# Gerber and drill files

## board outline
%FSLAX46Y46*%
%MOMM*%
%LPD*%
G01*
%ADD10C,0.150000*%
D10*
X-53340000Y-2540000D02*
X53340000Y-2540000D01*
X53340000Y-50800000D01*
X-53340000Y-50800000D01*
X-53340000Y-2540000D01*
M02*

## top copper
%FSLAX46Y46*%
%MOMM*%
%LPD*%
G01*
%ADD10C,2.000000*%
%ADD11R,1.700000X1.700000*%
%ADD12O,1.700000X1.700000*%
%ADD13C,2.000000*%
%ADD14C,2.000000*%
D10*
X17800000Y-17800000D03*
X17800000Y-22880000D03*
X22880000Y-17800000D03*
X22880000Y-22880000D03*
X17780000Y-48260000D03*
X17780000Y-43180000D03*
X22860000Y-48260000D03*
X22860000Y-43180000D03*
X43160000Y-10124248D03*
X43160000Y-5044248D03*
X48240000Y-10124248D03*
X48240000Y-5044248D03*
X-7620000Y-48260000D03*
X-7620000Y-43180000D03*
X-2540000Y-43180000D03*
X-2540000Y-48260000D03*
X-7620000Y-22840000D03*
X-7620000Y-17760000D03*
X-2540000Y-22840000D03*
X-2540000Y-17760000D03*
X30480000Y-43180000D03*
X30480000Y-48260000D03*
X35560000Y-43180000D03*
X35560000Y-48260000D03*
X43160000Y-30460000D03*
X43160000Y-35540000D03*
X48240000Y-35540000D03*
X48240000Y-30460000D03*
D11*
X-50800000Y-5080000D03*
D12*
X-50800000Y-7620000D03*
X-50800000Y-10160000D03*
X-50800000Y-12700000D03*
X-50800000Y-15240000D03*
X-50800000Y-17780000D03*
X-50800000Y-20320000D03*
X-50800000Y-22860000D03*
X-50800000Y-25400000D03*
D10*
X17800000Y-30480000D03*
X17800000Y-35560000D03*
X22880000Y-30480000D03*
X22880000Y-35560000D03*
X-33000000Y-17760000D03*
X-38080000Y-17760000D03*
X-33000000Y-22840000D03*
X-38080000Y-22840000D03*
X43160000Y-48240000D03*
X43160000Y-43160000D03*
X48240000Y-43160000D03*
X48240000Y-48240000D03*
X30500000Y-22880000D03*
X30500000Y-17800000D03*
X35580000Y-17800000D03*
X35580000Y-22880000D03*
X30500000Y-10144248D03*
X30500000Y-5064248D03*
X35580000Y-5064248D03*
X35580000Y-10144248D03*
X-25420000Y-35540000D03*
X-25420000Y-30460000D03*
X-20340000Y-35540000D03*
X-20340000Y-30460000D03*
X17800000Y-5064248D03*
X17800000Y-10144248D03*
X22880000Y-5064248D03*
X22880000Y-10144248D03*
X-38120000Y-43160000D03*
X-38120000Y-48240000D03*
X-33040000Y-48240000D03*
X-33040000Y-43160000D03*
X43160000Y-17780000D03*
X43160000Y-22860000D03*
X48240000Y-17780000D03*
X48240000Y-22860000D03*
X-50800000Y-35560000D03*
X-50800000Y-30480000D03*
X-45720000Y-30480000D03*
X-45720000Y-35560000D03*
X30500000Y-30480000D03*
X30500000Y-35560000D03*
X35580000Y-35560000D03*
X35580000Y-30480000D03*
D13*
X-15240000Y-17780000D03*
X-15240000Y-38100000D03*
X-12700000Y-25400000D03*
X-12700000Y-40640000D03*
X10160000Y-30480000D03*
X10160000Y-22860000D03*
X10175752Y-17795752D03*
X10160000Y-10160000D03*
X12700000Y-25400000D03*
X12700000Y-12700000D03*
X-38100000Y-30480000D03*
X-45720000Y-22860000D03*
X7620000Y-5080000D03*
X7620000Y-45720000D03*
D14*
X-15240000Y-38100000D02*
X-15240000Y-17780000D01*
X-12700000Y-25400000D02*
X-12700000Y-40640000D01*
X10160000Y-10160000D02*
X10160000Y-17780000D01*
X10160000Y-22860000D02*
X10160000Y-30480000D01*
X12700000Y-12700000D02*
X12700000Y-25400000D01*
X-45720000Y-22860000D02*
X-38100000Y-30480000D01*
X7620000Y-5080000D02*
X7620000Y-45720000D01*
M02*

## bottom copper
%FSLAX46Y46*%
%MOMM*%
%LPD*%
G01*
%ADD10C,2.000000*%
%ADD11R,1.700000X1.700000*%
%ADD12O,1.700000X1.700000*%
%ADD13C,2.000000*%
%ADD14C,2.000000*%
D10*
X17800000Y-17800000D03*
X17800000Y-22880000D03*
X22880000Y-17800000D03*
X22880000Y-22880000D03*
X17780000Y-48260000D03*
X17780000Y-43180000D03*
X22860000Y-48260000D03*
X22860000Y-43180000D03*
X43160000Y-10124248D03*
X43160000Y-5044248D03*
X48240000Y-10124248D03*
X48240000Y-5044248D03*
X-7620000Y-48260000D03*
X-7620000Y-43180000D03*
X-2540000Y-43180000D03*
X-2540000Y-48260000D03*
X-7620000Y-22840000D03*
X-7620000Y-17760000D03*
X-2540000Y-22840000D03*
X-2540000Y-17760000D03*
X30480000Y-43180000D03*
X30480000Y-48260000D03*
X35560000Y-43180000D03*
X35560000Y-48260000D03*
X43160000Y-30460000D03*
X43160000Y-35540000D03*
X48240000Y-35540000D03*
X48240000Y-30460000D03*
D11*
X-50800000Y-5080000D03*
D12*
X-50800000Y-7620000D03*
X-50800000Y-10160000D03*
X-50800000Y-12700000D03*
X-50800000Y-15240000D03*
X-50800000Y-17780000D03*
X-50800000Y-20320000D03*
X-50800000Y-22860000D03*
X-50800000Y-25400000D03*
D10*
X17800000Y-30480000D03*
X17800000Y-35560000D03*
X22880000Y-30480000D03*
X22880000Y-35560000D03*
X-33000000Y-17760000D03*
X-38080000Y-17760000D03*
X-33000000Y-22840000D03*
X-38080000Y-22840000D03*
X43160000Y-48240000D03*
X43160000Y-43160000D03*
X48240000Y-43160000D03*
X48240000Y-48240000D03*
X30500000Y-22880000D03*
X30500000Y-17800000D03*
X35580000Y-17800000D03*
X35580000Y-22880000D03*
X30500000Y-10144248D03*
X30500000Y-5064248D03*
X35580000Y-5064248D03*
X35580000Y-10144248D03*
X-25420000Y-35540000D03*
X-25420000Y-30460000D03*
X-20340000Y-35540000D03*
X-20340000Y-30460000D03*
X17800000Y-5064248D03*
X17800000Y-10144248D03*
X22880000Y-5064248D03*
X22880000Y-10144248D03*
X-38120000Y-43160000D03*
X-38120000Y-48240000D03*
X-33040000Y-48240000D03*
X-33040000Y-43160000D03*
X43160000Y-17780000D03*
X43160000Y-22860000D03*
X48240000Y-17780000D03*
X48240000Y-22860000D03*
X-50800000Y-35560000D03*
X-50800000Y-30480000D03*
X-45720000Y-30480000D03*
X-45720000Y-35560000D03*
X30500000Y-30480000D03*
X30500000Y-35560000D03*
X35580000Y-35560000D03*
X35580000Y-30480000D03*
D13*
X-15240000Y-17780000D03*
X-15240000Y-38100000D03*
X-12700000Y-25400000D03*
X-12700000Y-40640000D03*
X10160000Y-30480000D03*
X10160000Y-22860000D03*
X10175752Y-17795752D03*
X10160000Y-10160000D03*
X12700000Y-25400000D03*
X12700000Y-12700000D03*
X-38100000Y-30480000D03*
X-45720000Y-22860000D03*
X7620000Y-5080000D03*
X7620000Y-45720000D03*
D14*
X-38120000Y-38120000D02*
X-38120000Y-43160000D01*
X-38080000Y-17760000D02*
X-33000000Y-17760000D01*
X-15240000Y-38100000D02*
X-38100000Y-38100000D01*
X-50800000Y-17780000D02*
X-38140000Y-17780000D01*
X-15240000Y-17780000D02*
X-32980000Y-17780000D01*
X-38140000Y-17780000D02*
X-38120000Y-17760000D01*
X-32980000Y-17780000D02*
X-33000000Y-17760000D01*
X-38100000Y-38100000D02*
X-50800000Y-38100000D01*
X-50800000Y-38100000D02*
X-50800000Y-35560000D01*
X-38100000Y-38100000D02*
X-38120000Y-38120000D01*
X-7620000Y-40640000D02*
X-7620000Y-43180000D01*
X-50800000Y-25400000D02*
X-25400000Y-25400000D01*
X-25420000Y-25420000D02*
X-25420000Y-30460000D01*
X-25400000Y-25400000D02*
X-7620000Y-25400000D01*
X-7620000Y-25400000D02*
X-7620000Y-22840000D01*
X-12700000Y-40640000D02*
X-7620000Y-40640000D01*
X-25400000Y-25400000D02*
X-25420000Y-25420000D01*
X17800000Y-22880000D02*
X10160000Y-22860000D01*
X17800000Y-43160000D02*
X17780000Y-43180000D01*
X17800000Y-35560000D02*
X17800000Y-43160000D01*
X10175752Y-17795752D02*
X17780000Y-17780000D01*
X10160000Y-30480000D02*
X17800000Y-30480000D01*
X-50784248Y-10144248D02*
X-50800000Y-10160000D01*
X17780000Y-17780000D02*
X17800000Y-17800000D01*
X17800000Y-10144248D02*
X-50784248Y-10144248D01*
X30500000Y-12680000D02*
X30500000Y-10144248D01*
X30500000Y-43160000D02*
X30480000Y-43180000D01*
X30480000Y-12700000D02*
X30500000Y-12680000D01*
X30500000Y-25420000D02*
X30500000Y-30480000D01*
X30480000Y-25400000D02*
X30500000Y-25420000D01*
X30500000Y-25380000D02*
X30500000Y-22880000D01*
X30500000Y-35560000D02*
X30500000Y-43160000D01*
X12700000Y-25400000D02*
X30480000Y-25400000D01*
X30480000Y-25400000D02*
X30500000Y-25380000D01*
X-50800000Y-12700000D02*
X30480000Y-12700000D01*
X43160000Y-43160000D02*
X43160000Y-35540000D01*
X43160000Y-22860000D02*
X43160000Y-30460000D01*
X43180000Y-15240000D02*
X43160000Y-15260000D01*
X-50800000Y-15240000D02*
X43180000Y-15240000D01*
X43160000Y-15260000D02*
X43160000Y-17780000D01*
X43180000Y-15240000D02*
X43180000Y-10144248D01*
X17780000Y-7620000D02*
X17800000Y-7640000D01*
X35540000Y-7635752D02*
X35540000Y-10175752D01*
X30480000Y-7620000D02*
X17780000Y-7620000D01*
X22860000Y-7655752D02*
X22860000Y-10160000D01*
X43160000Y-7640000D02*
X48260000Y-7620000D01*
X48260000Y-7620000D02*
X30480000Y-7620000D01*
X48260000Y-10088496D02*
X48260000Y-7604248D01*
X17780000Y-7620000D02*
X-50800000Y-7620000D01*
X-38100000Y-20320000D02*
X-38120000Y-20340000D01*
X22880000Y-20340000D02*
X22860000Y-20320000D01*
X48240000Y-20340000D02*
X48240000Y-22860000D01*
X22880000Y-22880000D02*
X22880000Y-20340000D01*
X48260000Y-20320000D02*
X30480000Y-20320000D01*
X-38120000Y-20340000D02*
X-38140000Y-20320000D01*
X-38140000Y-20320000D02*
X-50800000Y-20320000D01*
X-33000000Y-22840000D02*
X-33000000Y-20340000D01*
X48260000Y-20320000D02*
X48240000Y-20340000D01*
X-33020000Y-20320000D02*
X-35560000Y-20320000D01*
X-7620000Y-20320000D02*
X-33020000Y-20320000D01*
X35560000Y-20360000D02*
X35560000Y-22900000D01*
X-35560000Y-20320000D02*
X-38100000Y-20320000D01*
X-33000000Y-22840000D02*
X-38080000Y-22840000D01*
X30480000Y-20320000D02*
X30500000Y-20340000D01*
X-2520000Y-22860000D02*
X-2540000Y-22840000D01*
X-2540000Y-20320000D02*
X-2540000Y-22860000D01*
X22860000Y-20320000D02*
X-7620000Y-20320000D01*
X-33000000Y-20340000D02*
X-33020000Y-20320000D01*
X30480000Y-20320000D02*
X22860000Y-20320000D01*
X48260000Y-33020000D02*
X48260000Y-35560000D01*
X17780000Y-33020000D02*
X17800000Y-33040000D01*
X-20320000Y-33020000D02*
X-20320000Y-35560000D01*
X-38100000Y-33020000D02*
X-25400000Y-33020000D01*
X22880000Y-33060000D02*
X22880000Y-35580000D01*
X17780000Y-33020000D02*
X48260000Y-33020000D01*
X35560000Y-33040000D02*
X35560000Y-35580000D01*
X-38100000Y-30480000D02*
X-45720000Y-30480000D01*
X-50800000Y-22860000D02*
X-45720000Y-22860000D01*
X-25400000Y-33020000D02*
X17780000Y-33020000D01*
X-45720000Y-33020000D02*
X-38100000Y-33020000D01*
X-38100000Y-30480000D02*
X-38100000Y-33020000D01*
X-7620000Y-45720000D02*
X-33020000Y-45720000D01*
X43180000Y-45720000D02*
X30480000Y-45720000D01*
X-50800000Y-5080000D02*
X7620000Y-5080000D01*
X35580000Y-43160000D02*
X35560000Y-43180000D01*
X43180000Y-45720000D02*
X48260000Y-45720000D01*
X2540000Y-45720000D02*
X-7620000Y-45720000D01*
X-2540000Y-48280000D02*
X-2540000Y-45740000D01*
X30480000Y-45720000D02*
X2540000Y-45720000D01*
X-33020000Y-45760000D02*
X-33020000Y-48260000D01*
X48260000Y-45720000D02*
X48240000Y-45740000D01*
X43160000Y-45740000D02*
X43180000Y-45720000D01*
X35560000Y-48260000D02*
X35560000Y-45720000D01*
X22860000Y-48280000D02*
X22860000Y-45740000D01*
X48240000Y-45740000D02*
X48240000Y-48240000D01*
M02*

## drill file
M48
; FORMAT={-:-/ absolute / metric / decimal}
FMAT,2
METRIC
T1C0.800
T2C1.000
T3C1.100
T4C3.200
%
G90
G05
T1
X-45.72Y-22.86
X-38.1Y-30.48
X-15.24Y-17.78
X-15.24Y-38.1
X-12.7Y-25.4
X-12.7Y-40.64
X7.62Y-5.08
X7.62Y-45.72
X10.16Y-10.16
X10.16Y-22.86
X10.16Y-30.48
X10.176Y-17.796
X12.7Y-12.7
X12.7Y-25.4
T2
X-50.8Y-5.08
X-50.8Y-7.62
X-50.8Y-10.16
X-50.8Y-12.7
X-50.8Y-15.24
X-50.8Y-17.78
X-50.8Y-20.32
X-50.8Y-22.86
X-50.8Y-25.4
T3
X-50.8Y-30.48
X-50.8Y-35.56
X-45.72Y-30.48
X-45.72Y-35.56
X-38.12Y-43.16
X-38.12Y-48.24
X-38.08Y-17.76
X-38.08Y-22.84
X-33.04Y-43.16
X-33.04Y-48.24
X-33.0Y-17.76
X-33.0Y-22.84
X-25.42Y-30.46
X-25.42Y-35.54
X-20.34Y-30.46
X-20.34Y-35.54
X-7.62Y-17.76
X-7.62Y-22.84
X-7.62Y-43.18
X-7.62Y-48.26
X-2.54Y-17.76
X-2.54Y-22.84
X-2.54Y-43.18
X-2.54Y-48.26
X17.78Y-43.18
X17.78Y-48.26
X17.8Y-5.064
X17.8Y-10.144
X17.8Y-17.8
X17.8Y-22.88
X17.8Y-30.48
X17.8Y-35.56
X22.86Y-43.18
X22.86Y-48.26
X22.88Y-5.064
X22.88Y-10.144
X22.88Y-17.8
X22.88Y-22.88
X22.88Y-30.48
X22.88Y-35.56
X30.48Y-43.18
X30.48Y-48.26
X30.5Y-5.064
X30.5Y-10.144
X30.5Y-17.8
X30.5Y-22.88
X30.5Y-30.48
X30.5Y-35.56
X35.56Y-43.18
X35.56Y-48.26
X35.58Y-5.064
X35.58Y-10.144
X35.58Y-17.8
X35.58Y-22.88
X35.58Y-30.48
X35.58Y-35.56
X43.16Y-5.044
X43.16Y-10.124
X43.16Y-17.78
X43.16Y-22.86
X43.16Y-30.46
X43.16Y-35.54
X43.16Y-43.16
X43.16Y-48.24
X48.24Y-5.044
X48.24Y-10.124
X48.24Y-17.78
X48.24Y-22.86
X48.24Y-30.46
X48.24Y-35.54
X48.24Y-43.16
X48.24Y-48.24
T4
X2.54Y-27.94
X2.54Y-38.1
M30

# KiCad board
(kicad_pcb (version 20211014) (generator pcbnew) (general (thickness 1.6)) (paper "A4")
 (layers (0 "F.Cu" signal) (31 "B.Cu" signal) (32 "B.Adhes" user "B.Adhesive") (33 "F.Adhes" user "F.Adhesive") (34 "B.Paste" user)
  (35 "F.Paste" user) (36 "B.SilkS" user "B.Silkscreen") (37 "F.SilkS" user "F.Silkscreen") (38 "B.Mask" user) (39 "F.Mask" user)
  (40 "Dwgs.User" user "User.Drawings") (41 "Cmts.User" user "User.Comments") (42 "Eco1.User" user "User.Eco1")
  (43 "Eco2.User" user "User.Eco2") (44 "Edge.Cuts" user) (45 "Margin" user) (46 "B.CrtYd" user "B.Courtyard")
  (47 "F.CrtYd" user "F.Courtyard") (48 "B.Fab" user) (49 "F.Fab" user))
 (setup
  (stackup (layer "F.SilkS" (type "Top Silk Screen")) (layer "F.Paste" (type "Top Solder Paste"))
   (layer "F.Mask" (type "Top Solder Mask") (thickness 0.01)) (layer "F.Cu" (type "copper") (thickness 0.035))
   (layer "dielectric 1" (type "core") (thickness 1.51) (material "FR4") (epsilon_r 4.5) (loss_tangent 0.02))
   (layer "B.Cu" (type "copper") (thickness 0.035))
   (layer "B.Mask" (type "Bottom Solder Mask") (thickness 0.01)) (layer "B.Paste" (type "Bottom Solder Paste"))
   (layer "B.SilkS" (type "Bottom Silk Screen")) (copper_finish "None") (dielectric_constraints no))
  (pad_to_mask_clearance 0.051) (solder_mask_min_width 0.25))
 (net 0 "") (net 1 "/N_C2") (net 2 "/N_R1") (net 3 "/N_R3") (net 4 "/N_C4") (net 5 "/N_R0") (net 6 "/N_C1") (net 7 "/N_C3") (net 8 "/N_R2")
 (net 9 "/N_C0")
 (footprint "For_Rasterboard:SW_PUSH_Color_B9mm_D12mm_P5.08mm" (layer "F.Cu") (at 17.8 17.8)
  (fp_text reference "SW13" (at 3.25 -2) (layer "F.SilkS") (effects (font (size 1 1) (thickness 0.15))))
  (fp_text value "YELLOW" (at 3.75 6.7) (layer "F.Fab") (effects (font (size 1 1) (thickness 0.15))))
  (pad "1" thru_hole circle (at 0 0 90) (size 2 2) (drill 1.1) (layers *.Cu *.Mask) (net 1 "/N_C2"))
  (pad "1" thru_hole circle (at 0 5.08 90) (size 2 2) (drill 1.1) (layers *.Cu *.Mask) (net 1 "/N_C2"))
  (pad "2" thru_hole circle (at 5.08 0 90) (size 2 2) (drill 1.1) (layers *.Cu *.Mask) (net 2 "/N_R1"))
  (pad "2" thru_hole circle (at 5.08 5.08 180) (size 2 2) (drill 1.1) (layers *.Cu *.Mask) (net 2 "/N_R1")))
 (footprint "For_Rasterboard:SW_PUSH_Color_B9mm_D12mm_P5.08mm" (layer "F.Cu") (at 17.78 43.18)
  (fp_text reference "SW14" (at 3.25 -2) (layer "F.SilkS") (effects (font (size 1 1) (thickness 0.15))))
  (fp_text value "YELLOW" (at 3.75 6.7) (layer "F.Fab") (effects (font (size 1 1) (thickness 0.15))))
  (pad "1" thru_hole circle (at 0 5.08 90) (size 2 2) (drill 1.1) (layers *.Cu *.Mask) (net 1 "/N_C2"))
  (pad "1" thru_hole circle (at 0 0 90) (size 2 2) (drill 1.1) (layers *.Cu *.Mask) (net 1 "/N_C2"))
  (pad "2" thru_hole circle (at 5.08 5.08 180) (size 2 2) (drill 1.1) (layers *.Cu *.Mask) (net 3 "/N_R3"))
  (pad "2" thru_hole circle (at 5.08 0 90) (size 2 2) (drill 1.1) (layers *.Cu *.Mask) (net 3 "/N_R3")))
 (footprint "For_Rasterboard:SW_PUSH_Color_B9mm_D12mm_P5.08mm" (layer "F.Cu") (at 43.16 5.044248)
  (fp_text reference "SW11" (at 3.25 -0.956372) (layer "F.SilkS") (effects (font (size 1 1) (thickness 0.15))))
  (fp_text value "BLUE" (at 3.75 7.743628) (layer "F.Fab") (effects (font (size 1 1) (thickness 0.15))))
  (pad "1" thru_hole circle (at 0 5.08 90) (size 2 2) (drill 1.1) (layers *.Cu *.Mask) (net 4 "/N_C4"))
  (pad "1" thru_hole circle (at 0 0 90) (size 2 2) (drill 1.1) (layers *.Cu *.Mask) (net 4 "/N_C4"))
  (pad "2" thru_hole circle (at 5.08 5.08 180) (size 2 2) (drill 1.1) (layers *.Cu *.Mask) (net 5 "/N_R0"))
  (pad "2" thru_hole circle (at 5.08 0 90) (size 2 2) (drill 1.1) (layers *.Cu *.Mask) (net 5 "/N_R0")))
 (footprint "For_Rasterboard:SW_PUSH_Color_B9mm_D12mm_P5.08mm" (layer "F.Cu") (at -7.62 43.18)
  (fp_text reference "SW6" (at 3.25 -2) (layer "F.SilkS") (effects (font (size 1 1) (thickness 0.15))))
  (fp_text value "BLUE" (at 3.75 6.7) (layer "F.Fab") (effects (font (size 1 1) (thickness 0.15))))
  (pad "1" thru_hole circle (at 0 5.08 90) (size 2 2) (drill 1.1) (layers *.Cu *.Mask) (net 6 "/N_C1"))
  (pad "1" thru_hole circle (at 0 0 90) (size 2 2) (drill 1.1) (layers *.Cu *.Mask) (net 6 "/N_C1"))
  (pad "2" thru_hole circle (at 5.08 0 90) (size 2 2) (drill 1.1) (layers *.Cu *.Mask) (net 3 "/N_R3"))
  (pad "2" thru_hole circle (at 5.08 5.08 180) (size 2 2) (drill 1.1) (layers *.Cu *.Mask) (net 3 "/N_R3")))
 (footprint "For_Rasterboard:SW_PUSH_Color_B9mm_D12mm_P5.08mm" (layer "F.Cu") (at -7.62 17.76)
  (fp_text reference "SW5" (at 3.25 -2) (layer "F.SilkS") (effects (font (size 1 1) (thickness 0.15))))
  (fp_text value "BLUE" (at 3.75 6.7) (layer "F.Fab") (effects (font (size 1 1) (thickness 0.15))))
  (pad "1" thru_hole circle (at 0 5.08 90) (size 2 2) (drill 1.1) (layers *.Cu *.Mask) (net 6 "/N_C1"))
  (pad "1" thru_hole circle (at 0 0 90) (size 2 2) (drill 1.1) (layers *.Cu *.Mask) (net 6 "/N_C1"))
  (pad "2" thru_hole circle (at 5.08 5.08 180) (size 2 2) (drill 1.1) (layers *.Cu *.Mask) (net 2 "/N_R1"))
  (pad "2" thru_hole circle (at 5.08 0 90) (size 2 2) (drill 1.1) (layers *.Cu *.Mask) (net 2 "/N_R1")))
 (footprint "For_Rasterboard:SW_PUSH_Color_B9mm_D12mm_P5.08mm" (layer "F.Cu") (at 30.48 43.18)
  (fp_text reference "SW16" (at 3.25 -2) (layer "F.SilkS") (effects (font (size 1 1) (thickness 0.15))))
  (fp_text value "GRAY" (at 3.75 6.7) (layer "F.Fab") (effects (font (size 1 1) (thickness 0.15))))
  (pad "1" thru_hole circle (at 0 0 90) (size 2 2) (drill 1.1) (layers *.Cu *.Mask) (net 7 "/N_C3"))
  (pad "1" thru_hole circle (at 0 5.08 90) (size 2 2) (drill 1.1) (layers *.Cu *.Mask) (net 7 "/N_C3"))
  (pad "2" thru_hole circle (at 5.08 0 90) (size 2 2) (drill 1.1) (layers *.Cu *.Mask) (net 3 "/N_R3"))
  (pad "2" thru_hole circle (at 5.08 5.08 180) (size 2 2) (drill 1.1) (layers *.Cu *.Mask) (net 3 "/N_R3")))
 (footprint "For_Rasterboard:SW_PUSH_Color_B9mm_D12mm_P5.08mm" (layer "F.Cu") (at 43.16 30.46)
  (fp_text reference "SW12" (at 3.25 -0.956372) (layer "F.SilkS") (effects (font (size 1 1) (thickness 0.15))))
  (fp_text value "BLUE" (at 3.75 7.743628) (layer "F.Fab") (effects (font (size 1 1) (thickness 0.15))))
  (pad "1" thru_hole circle (at 0 0 90) (size 2 2) (drill 1.1) (layers *.Cu *.Mask) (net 4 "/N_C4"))
  (pad "1" thru_hole circle (at 0 5.08 90) (size 2 2) (drill 1.1) (layers *.Cu *.Mask) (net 4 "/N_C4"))
  (pad "2" thru_hole circle (at 5.08 5.08 180) (size 2 2) (drill 1.1) (layers *.Cu *.Mask) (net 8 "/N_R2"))
  (pad "2" thru_hole circle (at 5.08 0 90) (size 2 2) (drill 1.1) (layers *.Cu *.Mask) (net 8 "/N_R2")))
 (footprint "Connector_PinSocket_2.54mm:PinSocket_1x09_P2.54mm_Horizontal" (layer "F.Cu") (at -50.8 5.08)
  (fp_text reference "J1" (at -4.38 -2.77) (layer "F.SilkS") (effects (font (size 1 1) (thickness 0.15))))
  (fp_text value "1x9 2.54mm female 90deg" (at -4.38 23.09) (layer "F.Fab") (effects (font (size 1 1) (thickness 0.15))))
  (pad "1" thru_hole rect (at 0 0) (size 1.7 1.7) (drill 1) (layers *.Cu *.Mask) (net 3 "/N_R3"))
  (pad "2" thru_hole oval (at 0 2.54) (size 1.7 1.7) (drill 1) (layers *.Cu *.Mask) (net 5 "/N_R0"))
  (pad "3" thru_hole oval (at 0 5.08) (size 1.7 1.7) (drill 1) (layers *.Cu *.Mask) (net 1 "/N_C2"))
  (pad "4" thru_hole oval (at 0 7.62) (size 1.7 1.7) (drill 1) (layers *.Cu *.Mask) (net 7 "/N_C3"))
  (pad "5" thru_hole oval (at 0 10.16) (size 1.7 1.7) (drill 1) (layers *.Cu *.Mask) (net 4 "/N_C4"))
  (pad "6" thru_hole oval (at 0 12.7) (size 1.7 1.7) (drill 1) (layers *.Cu *.Mask) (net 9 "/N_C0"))
  (pad "7" thru_hole oval (at 0 15.24) (size 1.7 1.7) (drill 1) (layers *.Cu *.Mask) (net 2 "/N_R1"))
  (pad "8" thru_hole oval (at 0 17.78) (size 1.7 1.7) (drill 1) (layers *.Cu *.Mask) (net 8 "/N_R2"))
  (pad "9" thru_hole oval (at 0 20.32) (size 1.7 1.7) (drill 1) (layers *.Cu *.Mask) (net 6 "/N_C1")))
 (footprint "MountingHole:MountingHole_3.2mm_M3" (layer "F.Cu") (at 2.54 27.94)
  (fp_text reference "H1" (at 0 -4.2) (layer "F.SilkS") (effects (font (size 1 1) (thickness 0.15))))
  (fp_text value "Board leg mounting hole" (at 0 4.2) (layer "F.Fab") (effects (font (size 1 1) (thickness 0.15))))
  (pad "" np_thru_hole circle (at 0 0) (size 3.2 3.2) (drill 3.2) (layers *.Cu *.Mask)))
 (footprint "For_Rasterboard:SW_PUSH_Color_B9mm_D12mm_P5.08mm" (layer "F.Cu") (at 17.8 30.48)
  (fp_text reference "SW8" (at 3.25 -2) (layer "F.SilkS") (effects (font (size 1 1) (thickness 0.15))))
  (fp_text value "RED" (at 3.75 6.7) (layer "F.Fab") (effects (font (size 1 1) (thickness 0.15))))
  (pad "1" thru_hole circle (at 0 0 90) (size 2 2) (drill 1.1) (layers *.Cu *.Mask) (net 1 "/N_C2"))
  (pad "1" thru_hole circle (at 0 5.08 90) (size 2 2) (drill 1.1) (layers *.Cu *.Mask) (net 1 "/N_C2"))
  (pad "2" thru_hole circle (at 5.08 0 90) (size 2 2) (drill 1.1) (layers *.Cu *.Mask) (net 8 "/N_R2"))
  (pad "2" thru_hole circle (at 5.08 5.08 180) (size 2 2) (drill 1.1) (layers *.Cu *.Mask) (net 8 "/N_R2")))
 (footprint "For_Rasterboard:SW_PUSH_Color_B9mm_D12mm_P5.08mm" (layer "F.Cu") (at -33 17.76 -90)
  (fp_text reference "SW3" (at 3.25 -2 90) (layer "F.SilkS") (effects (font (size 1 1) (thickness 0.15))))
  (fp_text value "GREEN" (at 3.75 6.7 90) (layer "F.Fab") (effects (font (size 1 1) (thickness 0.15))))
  (pad "1" thru_hole circle (at 0 0) (size 2 2) (drill 1.1) (layers *.Cu *.Mask) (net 9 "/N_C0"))
  (pad "1" thru_hole circle (at 0 5.08) (size 2 2) (drill 1.1) (layers *.Cu *.Mask) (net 9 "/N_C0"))
  (pad "2" thru_hole circle (at 5.08 0) (size 2 2) (drill 1.1) (layers *.Cu *.Mask) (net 2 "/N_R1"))
  (pad "2" thru_hole circle (at 5.08 5.08 90) (size 2 2) (drill 1.1) (layers *.Cu *.Mask) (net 2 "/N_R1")))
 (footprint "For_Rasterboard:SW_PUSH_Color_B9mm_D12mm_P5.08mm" (layer "F.Cu") (at 43.16 43.16)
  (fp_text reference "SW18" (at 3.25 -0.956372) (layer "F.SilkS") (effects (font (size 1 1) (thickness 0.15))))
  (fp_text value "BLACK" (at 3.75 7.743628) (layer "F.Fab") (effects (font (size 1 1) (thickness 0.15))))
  (pad "1" thru_hole circle (at 0 5.08 90) (size 2 2) (drill 1.1) (layers *.Cu *.Mask) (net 4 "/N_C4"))
  (pad "1" thru_hole circle (at 0 0 90) (size 2 2) (drill 1.1) (layers *.Cu *.Mask) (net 4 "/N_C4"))
  (pad "2" thru_hole circle (at 5.08 0 90) (size 2 2) (drill 1.1) (layers *.Cu *.Mask) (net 3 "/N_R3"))
  (pad "2" thru_hole circle (at 5.08 5.08 180) (size 2 2) (drill 1.1) (layers *.Cu *.Mask) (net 3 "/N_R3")))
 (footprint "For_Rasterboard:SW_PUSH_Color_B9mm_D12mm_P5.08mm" (layer "F.Cu") (at 30.5 17.8)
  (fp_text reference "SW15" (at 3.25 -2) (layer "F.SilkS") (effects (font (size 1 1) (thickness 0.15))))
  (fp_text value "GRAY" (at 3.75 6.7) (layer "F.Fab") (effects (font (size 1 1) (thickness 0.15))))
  (pad "1" thru_hole circle (at 0 5.08 90) (size 2 2) (drill 1.1) (layers *.Cu *.Mask) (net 7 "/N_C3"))
  (pad "1" thru_hole circle (at 0 0 90) (size 2 2) (drill 1.1) (layers *.Cu *.Mask) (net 7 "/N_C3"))
  (pad "2" thru_hole circle (at 5.08 0 90) (size 2 2) (drill 1.1) (layers *.Cu *.Mask) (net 2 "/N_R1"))
  (pad "2" thru_hole circle (at 5.08 5.08 180) (size 2 2) (drill 1.1) (layers *.Cu *.Mask) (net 2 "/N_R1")))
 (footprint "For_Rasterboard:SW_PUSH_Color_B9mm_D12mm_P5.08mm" (layer "F.Cu") (at 30.5 5.064248)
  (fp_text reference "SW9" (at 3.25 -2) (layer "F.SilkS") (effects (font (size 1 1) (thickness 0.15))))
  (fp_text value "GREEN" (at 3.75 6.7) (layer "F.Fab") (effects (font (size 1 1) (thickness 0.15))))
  (pad "1" thru_hole circle (at 0 5.08 90) (size 2 2) (drill 1.1) (layers *.Cu *.Mask) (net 7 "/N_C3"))
  (pad "1" thru_hole circle (at 0 0 90) (size 2 2) (drill 1.1) (layers *.Cu *.Mask) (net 7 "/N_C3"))
  (pad "2" thru_hole circle (at 5.08 0 90) (size 2 2) (drill 1.1) (layers *.Cu *.Mask) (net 5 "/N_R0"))
  (pad "2" thru_hole circle (at 5.08 5.08 180) (size 2 2) (drill 1.1) (layers *.Cu *.Mask) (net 5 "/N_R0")))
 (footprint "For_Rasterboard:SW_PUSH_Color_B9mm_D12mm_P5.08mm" (layer "F.Cu") (at -25.42 30.46)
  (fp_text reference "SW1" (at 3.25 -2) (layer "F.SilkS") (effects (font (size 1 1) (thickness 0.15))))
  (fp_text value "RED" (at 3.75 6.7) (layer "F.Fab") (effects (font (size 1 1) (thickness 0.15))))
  (pad "1" thru_hole circle (at 0 5.08 90) (size 2 2) (drill 1.1) (layers *.Cu *.Mask) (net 6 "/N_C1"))
  (pad "1" thru_hole circle (at 0 0 90) (size 2 2) (drill 1.1) (layers *.Cu *.Mask) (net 6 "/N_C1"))
  (pad "2" thru_hole circle (at 5.08 5.08 180) (size 2 2) (drill 1.1) (layers *.Cu *.Mask) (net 8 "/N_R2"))
  (pad "2" thru_hole circle (at 5.08 0 90) (size 2 2) (drill 1.1) (layers *.Cu *.Mask) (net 8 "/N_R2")))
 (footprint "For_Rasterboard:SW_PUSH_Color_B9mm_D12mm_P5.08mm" (layer "F.Cu") (at 17.8 5.064248)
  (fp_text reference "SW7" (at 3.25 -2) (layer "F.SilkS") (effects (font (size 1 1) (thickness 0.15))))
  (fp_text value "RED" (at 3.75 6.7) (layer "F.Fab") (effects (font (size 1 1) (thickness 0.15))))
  (pad "1" thru_hole circle (at 0 0 90) (size 2 2) (drill 1.1) (layers *.Cu *.Mask) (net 1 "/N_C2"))
  (pad "1" thru_hole circle (at 0 5.08 90) (size 2 2) (drill 1.1) (layers *.Cu *.Mask) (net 1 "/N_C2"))
  (pad "2" thru_hole circle (at 5.08 0 90) (size 2 2) (drill 1.1) (layers *.Cu *.Mask) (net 5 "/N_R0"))
  (pad "2" thru_hole circle (at 5.08 5.08 180) (size 2 2) (drill 1.1) (layers *.Cu *.Mask) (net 5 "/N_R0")))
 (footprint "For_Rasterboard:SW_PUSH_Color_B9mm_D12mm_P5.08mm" (layer "F.Cu") (at -38.12 43.16)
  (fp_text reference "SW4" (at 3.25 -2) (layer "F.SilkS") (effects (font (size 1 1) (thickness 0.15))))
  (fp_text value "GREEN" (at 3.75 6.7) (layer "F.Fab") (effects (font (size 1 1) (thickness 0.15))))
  (pad "1" thru_hole circle (at 0 0 90) (size 2 2) (drill 1.1) (layers *.Cu *.Mask) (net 9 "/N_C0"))
  (pad "1" thru_hole circle (at 0 5.08 90) (size 2 2) (drill 1.1) (layers *.Cu *.Mask) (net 9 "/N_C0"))
  (pad "2" thru_hole circle (at 5.08 5.08 180) (size 2 2) (drill 1.1) (layers *.Cu *.Mask) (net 3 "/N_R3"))
  (pad "2" thru_hole circle (at 5.08 0 90) (size 2 2) (drill 1.1) (layers *.Cu *.Mask) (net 3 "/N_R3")))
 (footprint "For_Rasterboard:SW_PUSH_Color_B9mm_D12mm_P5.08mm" (layer "F.Cu") (at 43.16 17.78)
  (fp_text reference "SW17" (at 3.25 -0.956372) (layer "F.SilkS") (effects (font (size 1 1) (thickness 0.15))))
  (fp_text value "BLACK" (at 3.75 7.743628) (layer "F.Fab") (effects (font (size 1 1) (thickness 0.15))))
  (pad "1" thru_hole circle (at 0 0 90) (size 2 2) (drill 1.1) (layers *.Cu *.Mask) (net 4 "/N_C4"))
  (pad "1" thru_hole circle (at 0 5.08 90) (size 2 2) (drill 1.1) (layers *.Cu *.Mask) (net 4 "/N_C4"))
  (pad "2" thru_hole circle (at 5.08 0 90) (size 2 2) (drill 1.1) (layers *.Cu *.Mask) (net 2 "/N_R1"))
  (pad "2" thru_hole circle (at 5.08 5.08 180) (size 2 2) (drill 1.1) (layers *.Cu *.Mask) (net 2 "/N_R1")))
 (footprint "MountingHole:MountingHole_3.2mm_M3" (layer "F.Cu") (at 2.54 38.1)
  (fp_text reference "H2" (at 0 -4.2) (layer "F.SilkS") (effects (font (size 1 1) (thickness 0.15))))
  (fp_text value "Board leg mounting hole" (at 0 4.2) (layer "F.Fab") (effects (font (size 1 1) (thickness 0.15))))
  (pad "" np_thru_hole circle (at 0 0) (size 3.2 3.2) (drill 3.2) (layers *.Cu *.Mask)))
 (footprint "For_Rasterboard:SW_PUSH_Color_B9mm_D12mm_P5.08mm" (layer "F.Cu") (at -50.8 30.48)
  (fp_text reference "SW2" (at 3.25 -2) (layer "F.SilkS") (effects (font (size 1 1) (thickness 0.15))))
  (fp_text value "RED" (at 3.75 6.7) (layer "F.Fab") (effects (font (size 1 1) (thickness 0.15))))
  (pad "1" thru_hole circle (at 0 5.08 90) (size 2 2) (drill 1.1) (layers *.Cu *.Mask) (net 9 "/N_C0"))
  (pad "1" thru_hole circle (at 0 0 90) (size 2 2) (drill 1.1) (layers *.Cu *.Mask) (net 9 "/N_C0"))
  (pad "2" thru_hole circle (at 5.08 0 90) (size 2 2) (drill 1.1) (layers *.Cu *.Mask) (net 8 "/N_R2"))
  (pad "2" thru_hole circle (at 5.08 5.08 180) (size 2 2) (drill 1.1) (layers *.Cu *.Mask) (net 8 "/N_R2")))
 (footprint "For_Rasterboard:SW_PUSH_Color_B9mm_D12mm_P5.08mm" (layer "F.Cu") (at 30.5 30.48)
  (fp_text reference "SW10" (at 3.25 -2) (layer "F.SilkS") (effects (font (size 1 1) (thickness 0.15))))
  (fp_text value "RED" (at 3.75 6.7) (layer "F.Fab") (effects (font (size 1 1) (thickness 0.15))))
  (pad "1" thru_hole circle (at 0 0 90) (size 2 2) (drill 1.1) (layers *.Cu *.Mask) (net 7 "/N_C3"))
  (pad "1" thru_hole circle (at 0 5.08 90) (size 2 2) (drill 1.1) (layers *.Cu *.Mask) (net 7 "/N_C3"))
  (pad "2" thru_hole circle (at 5.08 5.08 180) (size 2 2) (drill 1.1) (layers *.Cu *.Mask) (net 8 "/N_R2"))
  (pad "2" thru_hole circle (at 5.08 0 90) (size 2 2) (drill 1.1) (layers *.Cu *.Mask) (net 8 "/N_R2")))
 (gr_rect (start -53.34 2.54) (end 53.34 50.8) (layer "Edge.Cuts") (width 0.15) (fill none))
 (segment (start -15.24 38.1) (end -15.24 17.78) (width 2) (layer "F.Cu") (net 9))
 (via (at -15.24 17.78) (size 2) (drill 0.8) (layers "F.Cu" "B.Cu") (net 9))
 (via (at -15.24 38.1) (size 2) (drill 0.8) (layers "F.Cu" "B.Cu") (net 9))
 (segment (start -38.12 38.12) (end -38.12 43.16) (width 2) (layer "B.Cu") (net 9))
 (segment (start -38.08 17.76) (end -33 17.76) (width 2) (layer "B.Cu") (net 9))
 (segment (start -15.24 38.1) (end -38.1 38.1) (width 2) (layer "B.Cu") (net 9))
 (segment (start -50.8 17.78) (end -38.14 17.78) (width 2) (layer "B.Cu") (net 9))
 (segment (start -15.24 17.78) (end -32.98 17.78) (width 2) (layer "B.Cu") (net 9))
 (segment (start -38.14 17.78) (end -38.12 17.76) (width 2) (layer "B.Cu") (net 9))
 (segment (start -32.98 17.78) (end -33 17.76) (width 2) (layer "B.Cu") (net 9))
 (segment (start -38.1 38.1) (end -50.8 38.1) (width 2) (layer "B.Cu") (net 9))
 (segment (start -50.8 38.1) (end -50.8 35.56) (width 2) (layer "B.Cu") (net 9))
 (segment (start -38.1 38.1) (end -38.12 38.12) (width 2) (layer "B.Cu") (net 9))
 (segment (start -12.7 25.4) (end -12.7 40.64) (width 2) (layer "F.Cu") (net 6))
 (via (at -12.7 25.4) (size 2) (drill 0.8) (layers "F.Cu" "B.Cu") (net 6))
 (via (at -12.7 40.64) (size 2) (drill 0.8) (layers "F.Cu" "B.Cu") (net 6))
 (segment (start -7.62 40.64) (end -7.62 43.18) (width 2) (layer "B.Cu") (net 6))
 (segment (start -50.8 25.4) (end -25.4 25.4) (width 2) (layer "B.Cu") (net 6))
 (segment (start -25.42 25.42) (end -25.42 30.46) (width 2) (layer "B.Cu") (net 6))
 (segment (start -25.4 25.4) (end -7.62 25.4) (width 2) (layer "B.Cu") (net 6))
 (segment (start -7.62 25.4) (end -7.62 22.84) (width 2) (layer "B.Cu") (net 6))
 (segment (start -12.7 40.64) (end -7.62 40.64) (width 2) (layer "B.Cu") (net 6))
 (segment (start -25.4 25.4) (end -25.42 25.42) (width 2) (layer "B.Cu") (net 6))
 (segment (start 10.16 10.16) (end 10.16 17.78) (width 2) (layer "F.Cu") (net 1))
 (segment (start 10.16 22.86) (end 10.16 30.48) (width 2) (layer "F.Cu") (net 1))
 (via (at 10.16 30.48) (size 2) (drill 0.8) (layers "F.Cu" "B.Cu") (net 1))
 (via (at 10.16 22.86) (size 2) (drill 0.8) (layers "F.Cu" "B.Cu") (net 1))
 (via (at 10.175752 17.795752) (size 2) (drill 0.8) (layers "F.Cu" "B.Cu") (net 1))
 (via (at 10.16 10.16) (size 2) (drill 0.8) (layers "F.Cu" "B.Cu") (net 1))
 (segment (start 17.8 22.88) (end 10.16 22.86) (width 2) (layer "B.Cu") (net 1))
 (segment (start 17.8 43.16) (end 17.78 43.18) (width 2) (layer "B.Cu") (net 1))
 (segment (start 17.8 35.56) (end 17.8 43.16) (width 2) (layer "B.Cu") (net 1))
 (segment (start 10.175752 17.795752) (end 17.78 17.78) (width 2) (layer "B.Cu") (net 1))
 (segment (start 10.16 30.48) (end 17.8 30.48) (width 2) (layer "B.Cu") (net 1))
 (segment (start -50.784248 10.144248) (end -50.8 10.16) (width 2) (layer "B.Cu") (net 1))
 (segment (start 17.78 17.78) (end 17.8 17.8) (width 2) (layer "B.Cu") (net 1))
 (segment (start 17.8 10.144248) (end -50.784248 10.144248) (width 2) (layer "B.Cu") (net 1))
 (segment (start 12.7 12.7) (end 12.7 25.4) (width 2) (layer "F.Cu") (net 7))
 (via (at 12.7 25.4) (size 2) (drill 0.8) (layers "F.Cu" "B.Cu") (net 7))
 (via (at 12.7 12.7) (size 2) (drill 0.8) (layers "F.Cu" "B.Cu") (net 7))
 (segment (start 30.5 12.68) (end 30.5 10.144248) (width 2) (layer "B.Cu") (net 7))
 (segment (start 30.5 43.16) (end 30.48 43.18) (width 2) (layer "B.Cu") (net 7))
 (segment (start 30.48 12.7) (end 30.5 12.68) (width 2) (layer "B.Cu") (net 7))
 (segment (start 30.5 25.42) (end 30.5 30.48) (width 2) (layer "B.Cu") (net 7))
 (segment (start 30.48 25.4) (end 30.5 25.42) (width 2) (layer "B.Cu") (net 7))
 (segment (start 30.5 25.38) (end 30.5 22.88) (width 2) (layer "B.Cu") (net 7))
 (segment (start 30.5 35.56) (end 30.5 43.16) (width 2) (layer "B.Cu") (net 7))
 (segment (start 12.7 25.4) (end 30.48 25.4) (width 2) (layer "B.Cu") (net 7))
 (segment (start 30.48 25.4) (end 30.5 25.38) (width 2) (layer "B.Cu") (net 7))
 (segment (start -50.8 12.7) (end 30.48 12.7) (width 2) (layer "B.Cu") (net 7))
 (segment (start 43.16 43.16) (end 43.16 35.54) (width 2) (layer "B.Cu") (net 4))
 (segment (start 43.16 22.86) (end 43.16 30.46) (width 2) (layer "B.Cu") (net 4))
 (segment (start 43.18 15.24) (end 43.16 15.26) (width 2) (layer "B.Cu") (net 4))
 (segment (start -50.8 15.24) (end 43.18 15.24) (width 2) (layer "B.Cu") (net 4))
 (segment (start 43.16 15.26) (end 43.16 17.78) (width 2) (layer "B.Cu") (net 4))
 (segment (start 43.18 15.24) (end 43.18 10.144248) (width 2) (layer "B.Cu") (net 4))
 (segment (start 17.78 7.62) (end 17.8 7.64) (width 2) (layer "B.Cu") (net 5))
 (segment (start 35.54 7.635752) (end 35.54 10.175752) (width 2) (layer "B.Cu") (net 5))
 (segment (start 30.48 7.62) (end 17.78 7.62) (width 2) (layer "B.Cu") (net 5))
 (segment (start 22.86 7.655752) (end 22.86 10.16) (width 2) (layer "B.Cu") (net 5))
 (segment (start 43.16 7.64) (end 48.26 7.62) (width 2) (layer "B.Cu") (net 5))
 (segment (start 48.26 7.62) (end 30.48 7.62) (width 2) (layer "B.Cu") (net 5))
 (segment (start 48.26 10.088496) (end 48.26 7.604248) (width 2) (layer "B.Cu") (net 5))
 (segment (start 17.78 7.62) (end -50.8 7.62) (width 2) (layer "B.Cu") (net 5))
 (segment (start -38.1 20.32) (end -38.12 20.34) (width 2) (layer "B.Cu") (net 2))
 (segment (start 22.88 20.34) (end 22.86 20.32) (width 2) (layer "B.Cu") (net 2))
 (segment (start 48.24 20.34) (end 48.24 22.86) (width 2) (layer "B.Cu") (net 2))
 (segment (start 22.88 22.88) (end 22.88 20.34) (width 2) (layer "B.Cu") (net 2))
 (segment (start 48.26 20.32) (end 30.48 20.32) (width 2) (layer "B.Cu") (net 2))
 (segment (start -38.12 20.34) (end -38.14 20.32) (width 2) (layer "B.Cu") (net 2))
 (segment (start -38.14 20.32) (end -50.8 20.32) (width 2) (layer "B.Cu") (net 2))
 (segment (start -33 22.84) (end -33 20.34) (width 2) (layer "B.Cu") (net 2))
 (segment (start 48.26 20.32) (end 48.24 20.34) (width 2) (layer "B.Cu") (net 2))
 (segment (start -33.02 20.32) (end -35.56 20.32) (width 2) (layer "B.Cu") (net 2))
 (segment (start -7.62 20.32) (end -33.02 20.32) (width 2) (layer "B.Cu") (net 2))
 (segment (start 35.56 20.36) (end 35.56 22.9) (width 2) (layer "B.Cu") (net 2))
 (segment (start -35.56 20.32) (end -38.1 20.32) (width 2) (layer "B.Cu") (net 2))
 (segment (start -33 22.84) (end -38.08 22.84) (width 2) (layer "B.Cu") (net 2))
 (segment (start 30.48 20.32) (end 30.5 20.34) (width 2) (layer "B.Cu") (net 2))
 (segment (start -2.52 22.86) (end -2.54 22.84) (width 2) (layer "B.Cu") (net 2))
 (segment (start -2.54 20.32) (end -2.54 22.86) (width 2) (layer "B.Cu") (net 2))
 (segment (start 22.86 20.32) (end -7.62 20.32) (width 2) (layer "B.Cu") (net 2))
 (segment (start -33 20.34) (end -33.02 20.32) (width 2) (layer "B.Cu") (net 2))
 (segment (start 30.48 20.32) (end 22.86 20.32) (width 2) (layer "B.Cu") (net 2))
 (segment (start -45.72 22.86) (end -38.1 30.48) (width 2) (layer "F.Cu") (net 8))
 (via (at -38.1 30.48) (size 2) (drill 0.8) (layers "F.Cu" "B.Cu") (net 8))
 (via (at -45.72 22.86) (size 2) (drill 0.8) (layers "F.Cu" "B.Cu") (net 8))
 (segment (start 48.26 33.02) (end 48.26 35.56) (width 2) (layer "B.Cu") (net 8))
 (segment (start 17.78 33.02) (end 17.8 33.04) (width 2) (layer "B.Cu") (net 8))
 (segment (start -20.32 33.02) (end -20.32 35.56) (width 2) (layer "B.Cu") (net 8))
 (segment (start -38.1 33.02) (end -25.4 33.02) (width 2) (layer "B.Cu") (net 8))
 (segment (start 22.88 33.06) (end 22.88 35.58) (width 2) (layer "B.Cu") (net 8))
 (segment (start 17.78 33.02) (end 48.26 33.02) (width 2) (layer "B.Cu") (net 8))
 (segment (start 35.56 33.04) (end 35.56 35.58) (width 2) (layer "B.Cu") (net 8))
 (segment (start -38.1 30.48) (end -45.72 30.48) (width 2) (layer "B.Cu") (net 8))
 (segment (start -50.8 22.86) (end -45.72 22.86) (width 2) (layer "B.Cu") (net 8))
 (segment (start -25.4 33.02) (end 17.78 33.02) (width 2) (layer "B.Cu") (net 8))
 (segment (start -45.72 33.02) (end -38.1 33.02) (width 2) (layer "B.Cu") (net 8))
 (segment (start -38.1 30.48) (end -38.1 33.02) (width 2) (layer "B.Cu") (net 8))
 (segment (start 7.62 5.08) (end 7.62 45.72) (width 2) (layer "F.Cu") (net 3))
 (via (at 7.62 5.08) (size 2) (drill 0.8) (layers "F.Cu" "B.Cu") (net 3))
 (via (at 7.62 45.72) (size 2) (drill 0.8) (layers "F.Cu" "B.Cu") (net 3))
 (segment (start -7.62 45.72) (end -33.02 45.72) (width 2) (layer "B.Cu") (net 3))
 (segment (start 43.18 45.72) (end 30.48 45.72) (width 2) (layer "B.Cu") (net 3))
 (segment (start -50.8 5.08) (end 7.62 5.08) (width 2) (layer "B.Cu") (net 3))
 (segment (start 35.58 43.16) (end 35.56 43.18) (width 2) (layer "B.Cu") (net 3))
 (segment (start 43.18 45.72) (end 48.26 45.72) (width 2) (layer "B.Cu") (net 3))
 (segment (start 2.54 45.72) (end -7.62 45.72) (width 2) (layer "B.Cu") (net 3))
 (segment (start -2.54 48.28) (end -2.54 45.74) (width 2) (layer "B.Cu") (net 3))
 (segment (start 30.48 45.72) (end 2.54 45.72) (width 2) (layer "B.Cu") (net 3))
 (segment (start -33.02 45.76) (end -33.02 48.26) (width 2) (layer "B.Cu") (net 3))
 (segment (start 48.26 45.72) (end 48.24 45.74) (width 2) (layer "B.Cu") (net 3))
 (segment (start 43.16 45.74) (end 43.18 45.72) (width 2) (layer "B.Cu") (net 3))
 (segment (start 35.56 48.26) (end 35.56 45.72) (width 2) (layer "B.Cu") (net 3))
 (segment (start 22.86 48.28) (end 22.86 45.74) (width 2) (layer "B.Cu") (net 3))
 (segment (start 48.24 45.74) (end 48.24 48.24) (width 2) (layer "B.Cu") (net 3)))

